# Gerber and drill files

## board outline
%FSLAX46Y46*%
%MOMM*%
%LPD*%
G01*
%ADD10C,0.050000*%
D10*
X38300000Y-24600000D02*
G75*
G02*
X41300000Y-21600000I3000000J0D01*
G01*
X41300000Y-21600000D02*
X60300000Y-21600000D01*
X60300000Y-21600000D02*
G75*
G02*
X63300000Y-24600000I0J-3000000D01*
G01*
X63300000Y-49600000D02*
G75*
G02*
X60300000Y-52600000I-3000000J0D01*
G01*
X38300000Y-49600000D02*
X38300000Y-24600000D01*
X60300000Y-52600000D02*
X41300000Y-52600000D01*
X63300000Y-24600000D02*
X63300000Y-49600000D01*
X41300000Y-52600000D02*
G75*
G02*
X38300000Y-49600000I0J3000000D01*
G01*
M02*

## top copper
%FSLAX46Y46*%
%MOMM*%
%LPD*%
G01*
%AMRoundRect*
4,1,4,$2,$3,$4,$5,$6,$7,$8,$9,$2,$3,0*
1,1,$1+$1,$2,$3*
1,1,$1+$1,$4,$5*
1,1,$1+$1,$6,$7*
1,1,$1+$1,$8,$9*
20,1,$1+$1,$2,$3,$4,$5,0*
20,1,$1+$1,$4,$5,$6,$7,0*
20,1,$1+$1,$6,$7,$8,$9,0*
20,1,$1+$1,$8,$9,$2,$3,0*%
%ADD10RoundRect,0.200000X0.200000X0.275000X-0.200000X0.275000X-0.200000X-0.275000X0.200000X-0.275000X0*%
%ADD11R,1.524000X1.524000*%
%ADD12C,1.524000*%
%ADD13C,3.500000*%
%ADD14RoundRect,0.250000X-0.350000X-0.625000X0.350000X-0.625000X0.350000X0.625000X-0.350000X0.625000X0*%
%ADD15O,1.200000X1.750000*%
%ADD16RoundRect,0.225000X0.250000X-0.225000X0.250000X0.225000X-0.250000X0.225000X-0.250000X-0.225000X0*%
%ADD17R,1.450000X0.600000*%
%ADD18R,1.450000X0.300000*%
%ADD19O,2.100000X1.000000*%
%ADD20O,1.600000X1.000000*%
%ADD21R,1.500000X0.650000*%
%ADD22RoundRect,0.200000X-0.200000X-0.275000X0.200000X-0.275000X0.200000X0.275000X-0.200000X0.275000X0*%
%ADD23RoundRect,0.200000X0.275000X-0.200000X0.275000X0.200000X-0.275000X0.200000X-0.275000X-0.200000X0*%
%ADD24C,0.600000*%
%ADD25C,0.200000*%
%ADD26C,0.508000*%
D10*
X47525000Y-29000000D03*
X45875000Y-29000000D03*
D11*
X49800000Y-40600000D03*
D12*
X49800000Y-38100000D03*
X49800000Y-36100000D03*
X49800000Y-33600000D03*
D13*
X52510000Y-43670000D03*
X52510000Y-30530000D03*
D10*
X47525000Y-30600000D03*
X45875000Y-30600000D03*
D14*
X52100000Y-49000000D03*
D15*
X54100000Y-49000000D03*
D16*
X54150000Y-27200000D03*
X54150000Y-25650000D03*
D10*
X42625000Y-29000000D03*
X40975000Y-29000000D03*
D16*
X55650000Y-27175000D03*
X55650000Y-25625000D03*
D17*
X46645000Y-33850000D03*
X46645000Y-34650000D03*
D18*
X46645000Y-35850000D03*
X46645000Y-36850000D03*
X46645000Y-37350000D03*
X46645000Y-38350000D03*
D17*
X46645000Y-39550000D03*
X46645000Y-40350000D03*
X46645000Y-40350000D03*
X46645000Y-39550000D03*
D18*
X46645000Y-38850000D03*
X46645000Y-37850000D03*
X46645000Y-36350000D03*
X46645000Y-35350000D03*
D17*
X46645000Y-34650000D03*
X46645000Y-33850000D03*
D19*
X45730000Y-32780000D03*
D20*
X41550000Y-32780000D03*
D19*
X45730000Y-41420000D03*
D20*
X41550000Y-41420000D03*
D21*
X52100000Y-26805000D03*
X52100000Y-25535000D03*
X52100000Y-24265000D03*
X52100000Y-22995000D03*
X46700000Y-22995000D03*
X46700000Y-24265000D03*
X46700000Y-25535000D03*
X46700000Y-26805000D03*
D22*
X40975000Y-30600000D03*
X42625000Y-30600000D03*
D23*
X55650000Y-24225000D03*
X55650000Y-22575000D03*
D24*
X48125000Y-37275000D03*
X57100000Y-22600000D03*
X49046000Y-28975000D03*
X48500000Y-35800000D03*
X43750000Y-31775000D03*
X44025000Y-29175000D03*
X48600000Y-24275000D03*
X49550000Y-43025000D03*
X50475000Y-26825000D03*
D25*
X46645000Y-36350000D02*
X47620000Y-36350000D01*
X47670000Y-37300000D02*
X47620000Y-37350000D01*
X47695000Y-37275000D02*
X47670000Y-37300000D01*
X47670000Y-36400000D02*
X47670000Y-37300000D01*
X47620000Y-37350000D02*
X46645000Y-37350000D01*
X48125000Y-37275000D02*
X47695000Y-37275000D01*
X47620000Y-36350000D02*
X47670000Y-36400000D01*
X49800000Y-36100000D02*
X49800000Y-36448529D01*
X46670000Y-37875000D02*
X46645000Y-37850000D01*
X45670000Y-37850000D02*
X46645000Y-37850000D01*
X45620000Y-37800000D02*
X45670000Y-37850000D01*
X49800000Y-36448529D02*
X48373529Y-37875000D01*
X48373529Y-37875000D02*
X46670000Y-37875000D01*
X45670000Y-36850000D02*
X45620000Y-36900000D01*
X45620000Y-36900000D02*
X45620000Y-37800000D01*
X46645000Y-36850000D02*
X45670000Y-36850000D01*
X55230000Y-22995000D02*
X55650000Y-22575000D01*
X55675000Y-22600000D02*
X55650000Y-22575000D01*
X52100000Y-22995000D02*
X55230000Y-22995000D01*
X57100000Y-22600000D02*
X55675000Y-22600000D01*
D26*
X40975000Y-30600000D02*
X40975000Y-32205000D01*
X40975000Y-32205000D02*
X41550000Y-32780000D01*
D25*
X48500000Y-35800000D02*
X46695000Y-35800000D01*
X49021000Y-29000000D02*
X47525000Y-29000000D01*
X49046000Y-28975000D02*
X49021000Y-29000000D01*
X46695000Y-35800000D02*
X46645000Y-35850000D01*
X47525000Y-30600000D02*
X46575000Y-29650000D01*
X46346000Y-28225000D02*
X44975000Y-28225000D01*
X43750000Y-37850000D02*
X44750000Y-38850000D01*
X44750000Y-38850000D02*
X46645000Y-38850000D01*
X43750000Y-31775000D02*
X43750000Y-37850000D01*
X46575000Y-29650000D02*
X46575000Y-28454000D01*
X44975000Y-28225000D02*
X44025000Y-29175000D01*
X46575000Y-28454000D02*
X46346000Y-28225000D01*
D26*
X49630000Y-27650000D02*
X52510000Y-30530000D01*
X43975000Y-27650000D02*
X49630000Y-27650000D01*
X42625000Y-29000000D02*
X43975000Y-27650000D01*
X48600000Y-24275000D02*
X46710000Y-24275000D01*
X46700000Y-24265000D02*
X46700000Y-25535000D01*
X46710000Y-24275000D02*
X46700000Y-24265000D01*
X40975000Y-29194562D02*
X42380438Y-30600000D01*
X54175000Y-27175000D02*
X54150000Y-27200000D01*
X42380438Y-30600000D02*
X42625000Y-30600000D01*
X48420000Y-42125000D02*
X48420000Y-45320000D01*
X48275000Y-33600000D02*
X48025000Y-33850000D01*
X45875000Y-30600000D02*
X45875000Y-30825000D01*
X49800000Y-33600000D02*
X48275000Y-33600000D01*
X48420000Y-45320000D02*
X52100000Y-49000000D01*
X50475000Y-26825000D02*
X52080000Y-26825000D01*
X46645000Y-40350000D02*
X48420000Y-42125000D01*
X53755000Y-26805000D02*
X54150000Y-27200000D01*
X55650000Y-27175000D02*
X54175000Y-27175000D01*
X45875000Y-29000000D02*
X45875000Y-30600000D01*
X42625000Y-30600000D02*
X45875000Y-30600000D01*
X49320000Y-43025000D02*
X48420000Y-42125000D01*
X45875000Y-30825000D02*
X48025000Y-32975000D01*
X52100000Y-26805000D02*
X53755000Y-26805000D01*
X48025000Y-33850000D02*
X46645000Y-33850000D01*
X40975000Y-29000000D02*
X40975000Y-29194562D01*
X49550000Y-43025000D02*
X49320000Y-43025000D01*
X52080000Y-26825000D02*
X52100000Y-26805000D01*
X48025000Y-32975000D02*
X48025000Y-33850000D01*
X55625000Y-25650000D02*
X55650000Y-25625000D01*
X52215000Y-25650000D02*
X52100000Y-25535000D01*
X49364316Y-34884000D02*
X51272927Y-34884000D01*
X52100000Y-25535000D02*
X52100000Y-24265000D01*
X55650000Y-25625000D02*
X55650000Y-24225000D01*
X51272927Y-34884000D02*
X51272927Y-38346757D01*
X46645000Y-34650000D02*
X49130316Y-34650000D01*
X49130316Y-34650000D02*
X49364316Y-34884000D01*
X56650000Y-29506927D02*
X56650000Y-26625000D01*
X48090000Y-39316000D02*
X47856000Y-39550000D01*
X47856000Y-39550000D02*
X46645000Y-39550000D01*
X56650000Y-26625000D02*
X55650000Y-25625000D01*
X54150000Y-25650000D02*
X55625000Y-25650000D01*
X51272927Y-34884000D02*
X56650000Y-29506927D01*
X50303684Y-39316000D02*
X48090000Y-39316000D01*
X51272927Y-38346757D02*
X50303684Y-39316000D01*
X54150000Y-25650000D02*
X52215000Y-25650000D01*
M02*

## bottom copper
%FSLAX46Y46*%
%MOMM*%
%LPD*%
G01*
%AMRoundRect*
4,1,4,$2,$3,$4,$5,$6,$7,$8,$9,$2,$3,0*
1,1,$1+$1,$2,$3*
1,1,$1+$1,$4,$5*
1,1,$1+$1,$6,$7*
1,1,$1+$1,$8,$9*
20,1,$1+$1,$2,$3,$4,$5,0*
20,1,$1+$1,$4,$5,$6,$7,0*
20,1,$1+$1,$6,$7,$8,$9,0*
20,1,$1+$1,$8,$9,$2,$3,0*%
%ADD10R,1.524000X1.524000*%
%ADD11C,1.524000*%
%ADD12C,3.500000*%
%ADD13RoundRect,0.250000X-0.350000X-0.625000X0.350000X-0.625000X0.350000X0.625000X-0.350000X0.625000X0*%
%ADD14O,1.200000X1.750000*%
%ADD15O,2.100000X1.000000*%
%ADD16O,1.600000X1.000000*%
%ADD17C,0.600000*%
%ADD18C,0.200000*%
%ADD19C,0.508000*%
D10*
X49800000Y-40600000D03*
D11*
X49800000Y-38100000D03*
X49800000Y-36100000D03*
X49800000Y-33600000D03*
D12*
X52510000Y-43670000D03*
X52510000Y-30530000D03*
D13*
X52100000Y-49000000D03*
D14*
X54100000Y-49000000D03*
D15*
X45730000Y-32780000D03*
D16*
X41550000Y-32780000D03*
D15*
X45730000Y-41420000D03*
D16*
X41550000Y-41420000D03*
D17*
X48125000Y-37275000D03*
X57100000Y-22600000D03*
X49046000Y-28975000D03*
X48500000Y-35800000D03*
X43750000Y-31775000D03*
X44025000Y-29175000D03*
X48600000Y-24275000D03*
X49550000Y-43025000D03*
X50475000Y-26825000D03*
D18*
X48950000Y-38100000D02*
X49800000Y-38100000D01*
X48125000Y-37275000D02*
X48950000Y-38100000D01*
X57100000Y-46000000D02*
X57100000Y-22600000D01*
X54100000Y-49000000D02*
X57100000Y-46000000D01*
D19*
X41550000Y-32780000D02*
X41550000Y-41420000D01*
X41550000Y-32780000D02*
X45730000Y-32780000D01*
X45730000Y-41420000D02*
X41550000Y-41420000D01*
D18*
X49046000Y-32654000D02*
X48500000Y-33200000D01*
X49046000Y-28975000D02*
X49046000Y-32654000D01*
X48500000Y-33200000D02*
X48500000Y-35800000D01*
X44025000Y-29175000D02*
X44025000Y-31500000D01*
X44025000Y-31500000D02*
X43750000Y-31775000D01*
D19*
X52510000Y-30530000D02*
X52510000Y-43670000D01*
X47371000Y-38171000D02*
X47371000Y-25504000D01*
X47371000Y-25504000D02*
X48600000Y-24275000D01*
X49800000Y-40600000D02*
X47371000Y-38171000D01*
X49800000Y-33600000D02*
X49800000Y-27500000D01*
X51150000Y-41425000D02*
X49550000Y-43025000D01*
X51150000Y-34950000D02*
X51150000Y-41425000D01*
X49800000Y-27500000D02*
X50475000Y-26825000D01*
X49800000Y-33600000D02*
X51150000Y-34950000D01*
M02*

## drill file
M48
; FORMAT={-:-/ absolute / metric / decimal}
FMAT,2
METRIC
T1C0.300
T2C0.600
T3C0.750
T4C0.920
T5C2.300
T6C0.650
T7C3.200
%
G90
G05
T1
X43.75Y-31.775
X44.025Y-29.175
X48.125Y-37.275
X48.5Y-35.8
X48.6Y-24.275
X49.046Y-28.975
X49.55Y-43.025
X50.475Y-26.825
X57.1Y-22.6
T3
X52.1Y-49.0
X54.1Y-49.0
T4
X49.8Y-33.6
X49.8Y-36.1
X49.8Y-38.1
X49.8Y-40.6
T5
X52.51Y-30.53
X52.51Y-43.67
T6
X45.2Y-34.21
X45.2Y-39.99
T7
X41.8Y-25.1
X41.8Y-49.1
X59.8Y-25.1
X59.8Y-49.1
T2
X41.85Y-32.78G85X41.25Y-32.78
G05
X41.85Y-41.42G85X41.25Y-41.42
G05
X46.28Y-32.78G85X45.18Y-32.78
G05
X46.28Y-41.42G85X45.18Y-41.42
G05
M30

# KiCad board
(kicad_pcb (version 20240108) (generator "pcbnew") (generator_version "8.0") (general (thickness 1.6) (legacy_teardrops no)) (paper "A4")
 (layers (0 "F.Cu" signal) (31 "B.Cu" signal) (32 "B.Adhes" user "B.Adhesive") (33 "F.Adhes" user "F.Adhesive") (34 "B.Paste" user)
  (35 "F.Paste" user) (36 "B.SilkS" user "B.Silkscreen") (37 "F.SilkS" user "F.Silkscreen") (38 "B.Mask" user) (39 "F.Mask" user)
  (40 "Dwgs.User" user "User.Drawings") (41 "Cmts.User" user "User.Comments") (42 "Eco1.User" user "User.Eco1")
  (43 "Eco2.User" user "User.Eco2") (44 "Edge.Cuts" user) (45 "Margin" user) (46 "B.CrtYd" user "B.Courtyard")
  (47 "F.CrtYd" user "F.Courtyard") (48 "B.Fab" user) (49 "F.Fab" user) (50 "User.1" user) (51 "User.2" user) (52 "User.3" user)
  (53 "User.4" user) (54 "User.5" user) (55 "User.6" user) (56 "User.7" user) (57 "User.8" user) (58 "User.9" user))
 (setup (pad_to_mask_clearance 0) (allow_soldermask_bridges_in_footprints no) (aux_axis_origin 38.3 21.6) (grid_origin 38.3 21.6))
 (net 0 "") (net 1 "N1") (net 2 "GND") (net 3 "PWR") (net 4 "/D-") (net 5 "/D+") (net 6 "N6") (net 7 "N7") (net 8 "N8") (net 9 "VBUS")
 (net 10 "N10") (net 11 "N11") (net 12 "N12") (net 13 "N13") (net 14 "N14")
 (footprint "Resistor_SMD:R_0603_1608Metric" (layer "F.Cu") (at 46.7 29 180)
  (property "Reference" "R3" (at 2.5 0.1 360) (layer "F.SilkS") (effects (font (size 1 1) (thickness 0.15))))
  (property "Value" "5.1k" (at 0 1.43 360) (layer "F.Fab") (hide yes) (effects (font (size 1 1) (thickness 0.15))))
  (pad "1" smd roundrect (at -0.825 0 180) (size 0.8 0.95) (layers "F.Cu" "F.Paste" "F.Mask") (roundrect_rratio 0.25) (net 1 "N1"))
  (pad "2" smd roundrect (at 0.825 0 180) (size 0.8 0.95) (layers "F.Cu" "F.Paste" "F.Mask") (roundrect_rratio 0.25) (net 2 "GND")))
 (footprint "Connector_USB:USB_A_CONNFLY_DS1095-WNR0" (layer "F.Cu") (at 49.8 40.6 90)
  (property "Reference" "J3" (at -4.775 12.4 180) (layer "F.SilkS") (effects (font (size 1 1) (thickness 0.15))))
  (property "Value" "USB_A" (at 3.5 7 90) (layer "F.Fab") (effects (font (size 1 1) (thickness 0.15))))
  (pad "1" thru_hole rect (at 0 0 90) (size 1.524 1.524) (drill 0.92) (layers "*.Cu" "*.Mask") (remove_unused_layers no) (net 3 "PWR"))
  (pad "2" thru_hole circle (at 2.5 0 90) (size 1.524 1.524) (drill 0.92) (layers "*.Cu" "*.Mask") (remove_unused_layers no) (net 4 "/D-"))
  (pad "3" thru_hole circle (at 4.5 0 90) (size 1.524 1.524) (drill 0.92) (layers "*.Cu" "*.Mask") (remove_unused_layers no) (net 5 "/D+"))
  (pad "4" thru_hole circle (at 7 0 90) (size 1.524 1.524) (drill 0.92) (layers "*.Cu" "*.Mask") (remove_unused_layers no) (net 2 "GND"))
  (pad "5" thru_hole circle (at -3.07 2.71 90) (size 3.5 3.5) (drill 2.3) (layers "*.Cu" "*.Mask") (remove_unused_layers no) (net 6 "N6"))
  (pad "5" thru_hole circle (at 10.07 2.71 90) (size 3.5 3.5) (drill 2.3) (layers "*.Cu" "*.Mask") (remove_unused_layers no) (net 6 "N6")))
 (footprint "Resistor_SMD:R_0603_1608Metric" (layer "F.Cu") (at 46.7 30.6 180)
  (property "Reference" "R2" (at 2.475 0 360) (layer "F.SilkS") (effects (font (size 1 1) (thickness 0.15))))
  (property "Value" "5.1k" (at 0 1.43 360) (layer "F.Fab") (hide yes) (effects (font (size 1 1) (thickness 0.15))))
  (pad "1" smd roundrect (at -0.825 0 180) (size 0.8 0.95) (layers "F.Cu" "F.Paste" "F.Mask") (roundrect_rratio 0.25) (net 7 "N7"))
  (pad "2" smd roundrect (at 0.825 0 180) (size 0.8 0.95) (layers "F.Cu" "F.Paste" "F.Mask") (roundrect_rratio 0.25) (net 2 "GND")))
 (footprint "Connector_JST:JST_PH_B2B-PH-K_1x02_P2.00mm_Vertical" (layer "F.Cu") (at 52.1 49)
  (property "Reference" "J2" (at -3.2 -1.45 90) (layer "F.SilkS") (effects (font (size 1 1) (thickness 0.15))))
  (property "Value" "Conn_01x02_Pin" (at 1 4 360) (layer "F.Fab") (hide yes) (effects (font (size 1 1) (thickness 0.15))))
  (pad "1" thru_hole roundrect (at 0 0) (size 1.2 1.75) (drill 0.75) (layers "*.Cu" "*.Mask") (remove_unused_layers no)
   (roundrect_rratio 0.208333) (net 2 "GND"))
  (pad "2" thru_hole oval (at 2 0) (size 1.2 1.75) (drill 0.75) (layers "*.Cu" "*.Mask") (remove_unused_layers no) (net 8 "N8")))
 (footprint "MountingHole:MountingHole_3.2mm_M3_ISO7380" (layer "F.Cu") (at 59.8 49.1)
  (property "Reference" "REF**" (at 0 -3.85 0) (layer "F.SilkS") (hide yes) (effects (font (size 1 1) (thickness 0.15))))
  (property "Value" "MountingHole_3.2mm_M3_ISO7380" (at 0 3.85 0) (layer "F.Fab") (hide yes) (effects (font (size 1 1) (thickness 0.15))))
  (pad "" np_thru_hole circle (at 0 0) (size 3.2 3.2) (drill 3.2) (layers "*.Cu" "*.Mask")))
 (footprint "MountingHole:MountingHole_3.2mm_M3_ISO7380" (layer "F.Cu") (at 59.8 25.1)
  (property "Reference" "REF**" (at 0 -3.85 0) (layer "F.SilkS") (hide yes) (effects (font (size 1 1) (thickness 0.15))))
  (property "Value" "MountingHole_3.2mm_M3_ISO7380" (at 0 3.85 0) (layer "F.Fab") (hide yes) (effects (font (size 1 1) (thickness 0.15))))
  (pad "" np_thru_hole circle (at 0 0) (size 3.2 3.2) (drill 3.2) (layers "*.Cu" "*.Mask")))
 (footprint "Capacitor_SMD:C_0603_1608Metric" (layer "F.Cu") (at 54.15 26.425 90)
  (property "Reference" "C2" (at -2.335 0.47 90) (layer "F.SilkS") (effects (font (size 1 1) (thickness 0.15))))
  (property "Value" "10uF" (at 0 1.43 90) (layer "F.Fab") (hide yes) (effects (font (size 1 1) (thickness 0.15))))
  (pad "1" smd roundrect (at -0.775 0 90) (size 0.9 0.95) (layers "F.Cu" "F.Paste" "F.Mask") (roundrect_rratio 0.25) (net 2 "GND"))
  (pad "2" smd roundrect (at 0.775 0 90) (size 0.9 0.95) (layers "F.Cu" "F.Paste" "F.Mask") (roundrect_rratio 0.25) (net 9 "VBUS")))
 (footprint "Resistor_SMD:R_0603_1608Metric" (layer "F.Cu") (at 41.8 29 180)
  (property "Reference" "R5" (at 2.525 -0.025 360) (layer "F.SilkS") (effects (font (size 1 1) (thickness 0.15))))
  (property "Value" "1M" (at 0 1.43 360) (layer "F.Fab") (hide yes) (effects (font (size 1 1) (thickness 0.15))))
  (pad "1" smd roundrect (at -0.825 0 180) (size 0.8 0.95) (layers "F.Cu" "F.Paste" "F.Mask") (roundrect_rratio 0.25) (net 6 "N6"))
  (pad "2" smd roundrect (at 0.825 0 180) (size 0.8 0.95) (layers "F.Cu" "F.Paste" "F.Mask") (roundrect_rratio 0.25) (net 2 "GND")))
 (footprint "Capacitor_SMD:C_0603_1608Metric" (layer "F.Cu") (at 55.65 26.4 90)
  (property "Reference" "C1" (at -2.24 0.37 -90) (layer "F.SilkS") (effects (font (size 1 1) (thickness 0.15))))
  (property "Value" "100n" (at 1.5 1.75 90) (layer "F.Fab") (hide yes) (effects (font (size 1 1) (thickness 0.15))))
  (pad "1" smd roundrect (at -0.775 0 90) (size 0.9 0.95) (layers "F.Cu" "F.Paste" "F.Mask") (roundrect_rratio 0.25) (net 2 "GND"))
  (pad "2" smd roundrect (at 0.775 0 90) (size 0.9 0.95) (layers "F.Cu" "F.Paste" "F.Mask") (roundrect_rratio 0.25) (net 9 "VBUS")))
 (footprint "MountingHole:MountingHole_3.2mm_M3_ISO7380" (layer "F.Cu") (at 41.8 25.1)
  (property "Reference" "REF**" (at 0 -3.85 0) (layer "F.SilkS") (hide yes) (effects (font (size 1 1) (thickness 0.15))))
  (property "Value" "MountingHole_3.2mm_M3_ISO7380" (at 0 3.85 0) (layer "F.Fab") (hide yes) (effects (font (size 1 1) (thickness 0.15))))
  (pad "" np_thru_hole circle (at 0 0) (size 3.2 3.2) (drill 3.2) (layers "*.Cu" "*.Mask")))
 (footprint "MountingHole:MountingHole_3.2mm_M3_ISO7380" (layer "F.Cu") (at 41.8 49.1)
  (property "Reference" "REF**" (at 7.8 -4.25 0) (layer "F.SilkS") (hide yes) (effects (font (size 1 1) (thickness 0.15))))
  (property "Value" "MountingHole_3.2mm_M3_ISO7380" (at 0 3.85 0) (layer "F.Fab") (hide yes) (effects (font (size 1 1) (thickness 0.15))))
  (pad "" np_thru_hole circle (at 0 0) (size 3.2 3.2) (drill 3.2) (layers "*.Cu" "*.Mask")))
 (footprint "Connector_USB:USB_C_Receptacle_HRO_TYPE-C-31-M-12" (layer "F.Cu") (at 42.6 37.1 -90)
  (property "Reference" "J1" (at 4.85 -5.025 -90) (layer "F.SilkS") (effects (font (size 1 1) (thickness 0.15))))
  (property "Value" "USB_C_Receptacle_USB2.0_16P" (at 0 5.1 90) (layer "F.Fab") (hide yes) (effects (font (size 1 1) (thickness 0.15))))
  (pad "" np_thru_hole circle (at -2.89 -2.6 270) (size 0.65 0.65) (drill 0.65) (layers "*.Cu" "*.Mask"))
  (pad "" np_thru_hole circle (at 2.89 -2.6 270) (size 0.65 0.65) (drill 0.65) (layers "*.Cu" "*.Mask"))
  (pad "A1" smd rect (at -3.25 -4.045 270) (size 0.6 1.45) (layers "F.Cu" "F.Paste" "F.Mask") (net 2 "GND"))
  (pad "A4" smd rect (at -2.45 -4.045 270) (size 0.6 1.45) (layers "F.Cu" "F.Paste" "F.Mask") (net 9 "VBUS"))
  (pad "A5" smd rect (at -1.25 -4.045 270) (size 0.3 1.45) (layers "F.Cu" "F.Paste" "F.Mask") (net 1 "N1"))
  (pad "A6" smd rect (at -0.25 -4.045 270) (size 0.3 1.45) (layers "F.Cu" "F.Paste" "F.Mask") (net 5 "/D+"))
  (pad "A7" smd rect (at 0.25 -4.045 270) (size 0.3 1.45) (layers "F.Cu" "F.Paste" "F.Mask") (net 4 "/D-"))
  (pad "A8" smd rect (at 1.25 -4.045 270) (size 0.3 1.45) (layers "F.Cu" "F.Paste" "F.Mask") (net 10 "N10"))
  (pad "A9" smd rect (at 2.45 -4.045 270) (size 0.6 1.45) (layers "F.Cu" "F.Paste" "F.Mask") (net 9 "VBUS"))
  (pad "A12" smd rect (at 3.25 -4.045 270) (size 0.6 1.45) (layers "F.Cu" "F.Paste" "F.Mask") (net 2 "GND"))
  (pad "B1" smd rect (at 3.25 -4.045 270) (size 0.6 1.45) (layers "F.Cu" "F.Paste" "F.Mask") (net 2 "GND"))
  (pad "B4" smd rect (at 2.45 -4.045 270) (size 0.6 1.45) (layers "F.Cu" "F.Paste" "F.Mask") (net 9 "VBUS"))
  (pad "B5" smd rect (at 1.75 -4.045 270) (size 0.3 1.45) (layers "F.Cu" "F.Paste" "F.Mask") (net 7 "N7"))
  (pad "B6" smd rect (at 0.75 -4.045 270) (size 0.3 1.45) (layers "F.Cu" "F.Paste" "F.Mask") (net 5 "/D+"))
  (pad "B7" smd rect (at -0.75 -4.045 270) (size 0.3 1.45) (layers "F.Cu" "F.Paste" "F.Mask") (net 4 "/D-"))
  (pad "B8" smd rect (at -1.75 -4.045 270) (size 0.3 1.45) (layers "F.Cu" "F.Paste" "F.Mask") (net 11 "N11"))
  (pad "B9" smd rect (at -2.45 -4.045 270) (size 0.6 1.45) (layers "F.Cu" "F.Paste" "F.Mask") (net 9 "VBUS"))
  (pad "B12" smd rect (at -3.25 -4.045 270) (size 0.6 1.45) (layers "F.Cu" "F.Paste" "F.Mask") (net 2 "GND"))
  (pad "S1" thru_hole oval (at -4.32 -3.13 270) (size 1 2.1) (drill oval 0.6 1.7) (layers "*.Cu" "*.Mask") (remove_unused_layers no)
   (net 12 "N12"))
  (pad "S1" thru_hole oval (at -4.32 1.05 270) (size 1 1.6) (drill oval 0.6 1.2) (layers "*.Cu" "*.Mask") (remove_unused_layers no)
   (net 12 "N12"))
  (pad "S1" thru_hole oval (at 4.32 -3.13 270) (size 1 2.1) (drill oval 0.6 1.7) (layers "*.Cu" "*.Mask") (remove_unused_layers no)
   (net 12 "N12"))
  (pad "S1" thru_hole oval (at 4.32 1.05 270) (size 1 1.6) (drill oval 0.6 1.2) (layers "*.Cu" "*.Mask") (remove_unused_layers no)
   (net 12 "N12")))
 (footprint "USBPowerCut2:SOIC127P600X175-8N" (layer "F.Cu") (at 49.4 24.9 180)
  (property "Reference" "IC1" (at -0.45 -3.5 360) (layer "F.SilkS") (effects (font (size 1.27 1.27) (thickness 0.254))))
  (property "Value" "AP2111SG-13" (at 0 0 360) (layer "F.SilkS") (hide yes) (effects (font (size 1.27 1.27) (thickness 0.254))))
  (pad "1" smd rect (at -2.7 -1.905 270) (size 0.65 1.5) (layers "F.Cu" "F.Paste" "F.Mask") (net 2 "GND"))
  (pad "2" smd rect (at -2.7 -0.635 270) (size 0.65 1.5) (layers "F.Cu" "F.Paste" "F.Mask") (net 9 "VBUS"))
  (pad "3" smd rect (at -2.7 0.635 270) (size 0.65 1.5) (layers "F.Cu" "F.Paste" "F.Mask") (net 9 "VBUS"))
  (pad "4" smd rect (at -2.7 1.905 270) (size 0.65 1.5) (layers "F.Cu" "F.Paste" "F.Mask") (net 8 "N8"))
  (pad "5" smd rect (at 2.7 1.905 270) (size 0.65 1.5) (layers "F.Cu" "F.Paste" "F.Mask") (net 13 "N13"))
  (pad "6" smd rect (at 2.7 0.635 270) (size 0.65 1.5) (layers "F.Cu" "F.Paste" "F.Mask") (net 3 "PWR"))
  (pad "7" smd rect (at 2.7 -0.635 270) (size 0.65 1.5) (layers "F.Cu" "F.Paste" "F.Mask") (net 3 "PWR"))
  (pad "8" smd rect (at 2.7 -1.905 270) (size 0.65 1.5) (layers "F.Cu" "F.Paste" "F.Mask") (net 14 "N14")))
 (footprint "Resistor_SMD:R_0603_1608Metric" (layer "F.Cu") (at 41.8 30.6)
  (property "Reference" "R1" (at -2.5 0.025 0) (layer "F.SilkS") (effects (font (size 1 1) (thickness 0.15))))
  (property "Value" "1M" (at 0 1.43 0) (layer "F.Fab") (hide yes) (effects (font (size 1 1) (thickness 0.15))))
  (pad "1" smd roundrect (at -0.825 0) (size 0.8 0.95) (layers "F.Cu" "F.Paste" "F.Mask") (roundrect_rratio 0.25) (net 12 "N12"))
  (pad "2" smd roundrect (at 0.825 0) (size 0.8 0.95) (layers "F.Cu" "F.Paste" "F.Mask") (roundrect_rratio 0.25) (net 2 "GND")))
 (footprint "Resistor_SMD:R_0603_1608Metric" (layer "F.Cu") (at 55.65 23.4 90)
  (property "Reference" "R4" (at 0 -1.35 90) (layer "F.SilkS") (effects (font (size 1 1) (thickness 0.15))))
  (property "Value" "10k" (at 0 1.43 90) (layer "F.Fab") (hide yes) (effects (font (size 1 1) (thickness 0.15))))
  (pad "1" smd roundrect (at -0.825 0 90) (size 0.8 0.95) (layers "F.Cu" "F.Paste" "F.Mask") (roundrect_rratio 0.25) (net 9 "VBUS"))
  (pad "2" smd roundrect (at 0.825 0 90) (size 0.8 0.95) (layers "F.Cu" "F.Paste" "F.Mask") (roundrect_rratio 0.25) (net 8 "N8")))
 (gr_arc (start 38.3 24.6) (mid 39.17868 22.47868) (end 41.3 21.6) (stroke (width 0.05) (type default)) (layer "Edge.Cuts"))
 (gr_line (start 41.3 21.6) (end 60.3 21.6) (stroke (width 0.05) (type default)) (layer "Edge.Cuts"))
 (gr_arc (start 60.3 21.6) (mid 62.42132 22.47868) (end 63.3 24.6) (stroke (width 0.05) (type default)) (layer "Edge.Cuts"))
 (gr_arc (start 63.3 49.6) (mid 62.42132 51.72132) (end 60.3 52.6) (stroke (width 0.05) (type default)) (layer "Edge.Cuts"))
 (gr_line (start 38.3 49.6) (end 38.3 24.6) (stroke (width 0.05) (type default)) (layer "Edge.Cuts"))
 (gr_line (start 60.3 52.6) (end 41.3 52.6) (stroke (width 0.05) (type default)) (layer "Edge.Cuts"))
 (gr_line (start 63.3 24.6) (end 63.3 49.6) (stroke (width 0.05) (type default)) (layer "Edge.Cuts"))
 (gr_arc (start 41.3 52.6) (mid 39.17868 51.72132) (end 38.3 49.6) (stroke (width 0.05) (type default)) (layer "Edge.Cuts"))
 (segment (start 46.645 36.35) (end 47.62 36.35) (width 0.2) (layer "F.Cu") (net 4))
 (segment (start 47.67 37.3) (end 47.62 37.35) (width 0.2) (layer "F.Cu") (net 4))
 (segment (start 47.695 37.275) (end 47.67 37.3) (width 0.2) (layer "F.Cu") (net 4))
 (segment (start 47.67 36.4) (end 47.67 37.3) (width 0.2) (layer "F.Cu") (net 4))
 (segment (start 47.62 37.35) (end 46.645 37.35) (width 0.2) (layer "F.Cu") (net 4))
 (segment (start 48.125 37.275) (end 47.695 37.275) (width 0.2) (layer "F.Cu") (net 4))
 (segment (start 47.62 36.35) (end 47.67 36.4) (width 0.2) (layer "F.Cu") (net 4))
 (via (at 48.125 37.275) (size 0.6) (drill 0.3) (layers "F.Cu" "B.Cu") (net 4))
 (segment (start 48.95 38.1) (end 49.8 38.1) (width 0.2) (layer "B.Cu") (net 4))
 (segment (start 48.125 37.275) (end 48.95 38.1) (width 0.2) (layer "B.Cu") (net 4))
 (segment (start 49.8 36.1) (end 49.8 36.448529) (width 0.2) (layer "F.Cu") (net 5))
 (segment (start 46.67 37.875) (end 46.645 37.85) (width 0.2) (layer "F.Cu") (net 5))
 (segment (start 45.67 37.85) (end 46.645 37.85) (width 0.2) (layer "F.Cu") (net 5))
 (segment (start 45.62 37.8) (end 45.67 37.85) (width 0.2) (layer "F.Cu") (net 5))
 (segment (start 49.8 36.448529) (end 48.373529 37.875) (width 0.2) (layer "F.Cu") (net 5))
 (segment (start 48.373529 37.875) (end 46.67 37.875) (width 0.2) (layer "F.Cu") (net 5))
 (segment (start 45.67 36.85) (end 45.62 36.9) (width 0.2) (layer "F.Cu") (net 5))
 (segment (start 45.62 36.9) (end 45.62 37.8) (width 0.2) (layer "F.Cu") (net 5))
 (segment (start 46.645 36.85) (end 45.67 36.85) (width 0.2) (layer "F.Cu") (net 5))
 (segment (start 55.23 22.995) (end 55.65 22.575) (width 0.2) (layer "F.Cu") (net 8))
 (segment (start 55.675 22.6) (end 55.65 22.575) (width 0.2) (layer "F.Cu") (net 8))
 (segment (start 52.1 22.995) (end 55.23 22.995) (width 0.2) (layer "F.Cu") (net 8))
 (segment (start 57.1 22.6) (end 55.675 22.6) (width 0.2) (layer "F.Cu") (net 8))
 (via (at 57.1 22.6) (size 0.6) (drill 0.3) (layers "F.Cu" "B.Cu") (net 8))
 (segment (start 57.1 46) (end 57.1 22.6) (width 0.2) (layer "B.Cu") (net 8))
 (segment (start 54.1 49) (end 57.1 46) (width 0.2) (layer "B.Cu") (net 8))
 (segment (start 40.975 30.6) (end 40.975 32.205) (width 0.508) (layer "F.Cu") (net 12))
 (segment (start 40.975 32.205) (end 41.55 32.78) (width 0.508) (layer "F.Cu") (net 12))
 (segment (start 41.55 32.78) (end 41.55 41.42) (width 0.508) (layer "B.Cu") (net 12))
 (segment (start 41.55 32.78) (end 45.73 32.78) (width 0.508) (layer "B.Cu") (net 12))
 (segment (start 45.73 41.42) (end 41.55 41.42) (width 0.508) (layer "B.Cu") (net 12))
 (segment (start 48.5 35.8) (end 46.695 35.8) (width 0.2) (layer "F.Cu") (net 1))
 (segment (start 49.021 29) (end 47.525 29) (width 0.2) (layer "F.Cu") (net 1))
 (segment (start 49.046 28.975) (end 49.021 29) (width 0.2) (layer "F.Cu") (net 1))
 (segment (start 46.695 35.8) (end 46.645 35.85) (width 0.2) (layer "F.Cu") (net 1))
 (via (at 49.046 28.975) (size 0.6) (drill 0.3) (layers "F.Cu" "B.Cu") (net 1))
 (via (at 48.5 35.8) (size 0.6) (drill 0.3) (layers "F.Cu" "B.Cu") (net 1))
 (segment (start 49.046 32.654) (end 48.5 33.2) (width 0.2) (layer "B.Cu") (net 1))
 (segment (start 49.046 28.975) (end 49.046 32.654) (width 0.2) (layer "B.Cu") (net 1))
 (segment (start 48.5 33.2) (end 48.5 35.8) (width 0.2) (layer "B.Cu") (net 1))
 (segment (start 47.525 30.6) (end 46.575 29.65) (width 0.2) (layer "F.Cu") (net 7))
 (segment (start 46.346 28.225) (end 44.975 28.225) (width 0.2) (layer "F.Cu") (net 7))
 (segment (start 43.75 37.85) (end 44.75 38.85) (width 0.2) (layer "F.Cu") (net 7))
 (segment (start 44.75 38.85) (end 46.645 38.85) (width 0.2) (layer "F.Cu") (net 7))
 (segment (start 43.75 31.775) (end 43.75 37.85) (width 0.2) (layer "F.Cu") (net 7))
 (segment (start 46.575 29.65) (end 46.575 28.454) (width 0.2) (layer "F.Cu") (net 7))
 (segment (start 44.975 28.225) (end 44.025 29.175) (width 0.2) (layer "F.Cu") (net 7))
 (segment (start 46.575 28.454) (end 46.346 28.225) (width 0.2) (layer "F.Cu") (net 7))
 (via (at 43.75 31.775) (size 0.6) (drill 0.3) (layers "F.Cu" "B.Cu") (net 7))
 (via (at 44.025 29.175) (size 0.6) (drill 0.3) (layers "F.Cu" "B.Cu") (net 7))
 (segment (start 44.025 29.175) (end 44.025 31.5) (width 0.2) (layer "B.Cu") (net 7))
 (segment (start 44.025 31.5) (end 43.75 31.775) (width 0.2) (layer "B.Cu") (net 7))
 (segment (start 49.63 27.65) (end 52.51 30.53) (width 0.508) (layer "F.Cu") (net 6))
 (segment (start 43.975 27.65) (end 49.63 27.65) (width 0.508) (layer "F.Cu") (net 6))
 (segment (start 42.625 29) (end 43.975 27.65) (width 0.508) (layer "F.Cu") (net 6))
 (segment (start 52.51 30.53) (end 52.51 43.67) (width 0.508) (layer "B.Cu") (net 6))
 (segment (start 48.6 24.275) (end 46.71 24.275) (width 0.508) (layer "F.Cu") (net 3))
 (segment (start 46.7 24.265) (end 46.7 25.535) (width 0.508) (layer "F.Cu") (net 3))
 (segment (start 46.71 24.275) (end 46.7 24.265) (width 0.508) (layer "F.Cu") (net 3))
 (via (at 48.6 24.275) (size 0.6) (drill 0.3) (layers "F.Cu" "B.Cu") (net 3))
 (segment (start 47.371 38.171) (end 47.371 25.504) (width 0.508) (layer "B.Cu") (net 3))
 (segment (start 47.371 25.504) (end 48.6 24.275) (width 0.508) (layer "B.Cu") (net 3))
 (segment (start 49.8 40.6) (end 47.371 38.171) (width 0.508) (layer "B.Cu") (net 3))
 (segment (start 40.975 29.194562) (end 42.380438 30.6) (width 0.508) (layer "F.Cu") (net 2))
 (segment (start 54.175 27.175) (end 54.15 27.2) (width 0.508) (layer "F.Cu") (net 2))
 (segment (start 42.380438 30.6) (end 42.625 30.6) (width 0.508) (layer "F.Cu") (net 2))
 (segment (start 48.42 42.125) (end 48.42 45.32) (width 0.508) (layer "F.Cu") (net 2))
 (segment (start 48.275 33.6) (end 48.025 33.85) (width 0.508) (layer "F.Cu") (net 2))
 (segment (start 45.875 30.6) (end 45.875 30.825) (width 0.508) (layer "F.Cu") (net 2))
 (segment (start 49.8 33.6) (end 48.275 33.6) (width 0.508) (layer "F.Cu") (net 2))
 (segment (start 48.42 45.32) (end 52.1 49) (width 0.508) (layer "F.Cu") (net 2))
 (segment (start 50.475 26.825) (end 52.08 26.825) (width 0.508) (layer "F.Cu") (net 2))
 (segment (start 46.645 40.35) (end 48.42 42.125) (width 0.508) (layer "F.Cu") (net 2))
 (segment (start 53.755 26.805) (end 54.15 27.2) (width 0.508) (layer "F.Cu") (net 2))
 (segment (start 55.65 27.175) (end 54.175 27.175) (width 0.508) (layer "F.Cu") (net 2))
 (segment (start 45.875 29) (end 45.875 30.6) (width 0.508) (layer "F.Cu") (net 2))
 (segment (start 42.625 30.6) (end 45.875 30.6) (width 0.508) (layer "F.Cu") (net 2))
 (segment (start 49.32 43.025) (end 48.42 42.125) (width 0.508) (layer "F.Cu") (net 2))
 (segment (start 45.875 30.825) (end 48.025 32.975) (width 0.508) (layer "F.Cu") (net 2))
 (segment (start 52.1 26.805) (end 53.755 26.805) (width 0.508) (layer "F.Cu") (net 2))
 (segment (start 48.025 33.85) (end 46.645 33.85) (width 0.508) (layer "F.Cu") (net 2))
 (segment (start 40.975 29) (end 40.975 29.194562) (width 0.508) (layer "F.Cu") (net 2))
 (segment (start 49.55 43.025) (end 49.32 43.025) (width 0.508) (layer "F.Cu") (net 2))
 (segment (start 52.08 26.825) (end 52.1 26.805) (width 0.508) (layer "F.Cu") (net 2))
 (segment (start 48.025 32.975) (end 48.025 33.85) (width 0.508) (layer "F.Cu") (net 2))
 (via (at 49.55 43.025) (size 0.6) (drill 0.3) (layers "F.Cu" "B.Cu") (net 2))
 (via (at 50.475 26.825) (size 0.6) (drill 0.3) (layers "F.Cu" "B.Cu") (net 2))
 (segment (start 49.8 33.6) (end 49.8 27.5) (width 0.508) (layer "B.Cu") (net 2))
 (segment (start 51.15 41.425) (end 49.55 43.025) (width 0.508) (layer "B.Cu") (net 2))
 (segment (start 51.15 34.95) (end 51.15 41.425) (width 0.508) (layer "B.Cu") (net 2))
 (segment (start 49.8 27.5) (end 50.475 26.825) (width 0.508) (layer "B.Cu") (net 2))
 (segment (start 49.8 33.6) (end 51.15 34.95) (width 0.508) (layer "B.Cu") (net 2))
 (segment (start 55.625 25.65) (end 55.65 25.625) (width 0.508) (layer "F.Cu") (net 9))
 (segment (start 52.215 25.65) (end 52.1 25.535) (width 0.508) (layer "F.Cu") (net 9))
 (segment (start 49.364316 34.884) (end 51.272927 34.884) (width 0.508) (layer "F.Cu") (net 9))
 (segment (start 52.1 25.535) (end 52.1 24.265) (width 0.508) (layer "F.Cu") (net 9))
 (segment (start 55.65 25.625) (end 55.65 24.225) (width 0.508) (layer "F.Cu") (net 9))
 (segment (start 51.272927 34.884) (end 51.272927 38.346757) (width 0.508) (layer "F.Cu") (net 9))
 (segment (start 46.645 34.65) (end 49.130316 34.65) (width 0.508) (layer "F.Cu") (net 9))
 (segment (start 49.130316 34.65) (end 49.364316 34.884) (width 0.508) (layer "F.Cu") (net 9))
 (segment (start 56.65 29.506927) (end 56.65 26.625) (width 0.508) (layer "F.Cu") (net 9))
 (segment (start 48.09 39.316) (end 47.856 39.55) (width 0.508) (layer "F.Cu") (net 9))
 (segment (start 47.856 39.55) (end 46.645 39.55) (width 0.508) (layer "F.Cu") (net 9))
 (segment (start 56.65 26.625) (end 55.65 25.625) (width 0.508) (layer "F.Cu") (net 9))
 (segment (start 54.15 25.65) (end 55.625 25.65) (width 0.508) (layer "F.Cu") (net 9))
 (segment (start 51.272927 34.884) (end 56.65 29.506927) (width 0.508) (layer "F.Cu") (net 9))
 (segment (start 50.303684 39.316) (end 48.09 39.316) (width 0.508) (layer "F.Cu") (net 9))
 (segment (start 51.272927 38.346757) (end 50.303684 39.316) (width 0.508) (layer "F.Cu") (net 9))
 (segment (start 54.15 25.65) (end 52.215 25.65) (width 0.508) (layer "F.Cu") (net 9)))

